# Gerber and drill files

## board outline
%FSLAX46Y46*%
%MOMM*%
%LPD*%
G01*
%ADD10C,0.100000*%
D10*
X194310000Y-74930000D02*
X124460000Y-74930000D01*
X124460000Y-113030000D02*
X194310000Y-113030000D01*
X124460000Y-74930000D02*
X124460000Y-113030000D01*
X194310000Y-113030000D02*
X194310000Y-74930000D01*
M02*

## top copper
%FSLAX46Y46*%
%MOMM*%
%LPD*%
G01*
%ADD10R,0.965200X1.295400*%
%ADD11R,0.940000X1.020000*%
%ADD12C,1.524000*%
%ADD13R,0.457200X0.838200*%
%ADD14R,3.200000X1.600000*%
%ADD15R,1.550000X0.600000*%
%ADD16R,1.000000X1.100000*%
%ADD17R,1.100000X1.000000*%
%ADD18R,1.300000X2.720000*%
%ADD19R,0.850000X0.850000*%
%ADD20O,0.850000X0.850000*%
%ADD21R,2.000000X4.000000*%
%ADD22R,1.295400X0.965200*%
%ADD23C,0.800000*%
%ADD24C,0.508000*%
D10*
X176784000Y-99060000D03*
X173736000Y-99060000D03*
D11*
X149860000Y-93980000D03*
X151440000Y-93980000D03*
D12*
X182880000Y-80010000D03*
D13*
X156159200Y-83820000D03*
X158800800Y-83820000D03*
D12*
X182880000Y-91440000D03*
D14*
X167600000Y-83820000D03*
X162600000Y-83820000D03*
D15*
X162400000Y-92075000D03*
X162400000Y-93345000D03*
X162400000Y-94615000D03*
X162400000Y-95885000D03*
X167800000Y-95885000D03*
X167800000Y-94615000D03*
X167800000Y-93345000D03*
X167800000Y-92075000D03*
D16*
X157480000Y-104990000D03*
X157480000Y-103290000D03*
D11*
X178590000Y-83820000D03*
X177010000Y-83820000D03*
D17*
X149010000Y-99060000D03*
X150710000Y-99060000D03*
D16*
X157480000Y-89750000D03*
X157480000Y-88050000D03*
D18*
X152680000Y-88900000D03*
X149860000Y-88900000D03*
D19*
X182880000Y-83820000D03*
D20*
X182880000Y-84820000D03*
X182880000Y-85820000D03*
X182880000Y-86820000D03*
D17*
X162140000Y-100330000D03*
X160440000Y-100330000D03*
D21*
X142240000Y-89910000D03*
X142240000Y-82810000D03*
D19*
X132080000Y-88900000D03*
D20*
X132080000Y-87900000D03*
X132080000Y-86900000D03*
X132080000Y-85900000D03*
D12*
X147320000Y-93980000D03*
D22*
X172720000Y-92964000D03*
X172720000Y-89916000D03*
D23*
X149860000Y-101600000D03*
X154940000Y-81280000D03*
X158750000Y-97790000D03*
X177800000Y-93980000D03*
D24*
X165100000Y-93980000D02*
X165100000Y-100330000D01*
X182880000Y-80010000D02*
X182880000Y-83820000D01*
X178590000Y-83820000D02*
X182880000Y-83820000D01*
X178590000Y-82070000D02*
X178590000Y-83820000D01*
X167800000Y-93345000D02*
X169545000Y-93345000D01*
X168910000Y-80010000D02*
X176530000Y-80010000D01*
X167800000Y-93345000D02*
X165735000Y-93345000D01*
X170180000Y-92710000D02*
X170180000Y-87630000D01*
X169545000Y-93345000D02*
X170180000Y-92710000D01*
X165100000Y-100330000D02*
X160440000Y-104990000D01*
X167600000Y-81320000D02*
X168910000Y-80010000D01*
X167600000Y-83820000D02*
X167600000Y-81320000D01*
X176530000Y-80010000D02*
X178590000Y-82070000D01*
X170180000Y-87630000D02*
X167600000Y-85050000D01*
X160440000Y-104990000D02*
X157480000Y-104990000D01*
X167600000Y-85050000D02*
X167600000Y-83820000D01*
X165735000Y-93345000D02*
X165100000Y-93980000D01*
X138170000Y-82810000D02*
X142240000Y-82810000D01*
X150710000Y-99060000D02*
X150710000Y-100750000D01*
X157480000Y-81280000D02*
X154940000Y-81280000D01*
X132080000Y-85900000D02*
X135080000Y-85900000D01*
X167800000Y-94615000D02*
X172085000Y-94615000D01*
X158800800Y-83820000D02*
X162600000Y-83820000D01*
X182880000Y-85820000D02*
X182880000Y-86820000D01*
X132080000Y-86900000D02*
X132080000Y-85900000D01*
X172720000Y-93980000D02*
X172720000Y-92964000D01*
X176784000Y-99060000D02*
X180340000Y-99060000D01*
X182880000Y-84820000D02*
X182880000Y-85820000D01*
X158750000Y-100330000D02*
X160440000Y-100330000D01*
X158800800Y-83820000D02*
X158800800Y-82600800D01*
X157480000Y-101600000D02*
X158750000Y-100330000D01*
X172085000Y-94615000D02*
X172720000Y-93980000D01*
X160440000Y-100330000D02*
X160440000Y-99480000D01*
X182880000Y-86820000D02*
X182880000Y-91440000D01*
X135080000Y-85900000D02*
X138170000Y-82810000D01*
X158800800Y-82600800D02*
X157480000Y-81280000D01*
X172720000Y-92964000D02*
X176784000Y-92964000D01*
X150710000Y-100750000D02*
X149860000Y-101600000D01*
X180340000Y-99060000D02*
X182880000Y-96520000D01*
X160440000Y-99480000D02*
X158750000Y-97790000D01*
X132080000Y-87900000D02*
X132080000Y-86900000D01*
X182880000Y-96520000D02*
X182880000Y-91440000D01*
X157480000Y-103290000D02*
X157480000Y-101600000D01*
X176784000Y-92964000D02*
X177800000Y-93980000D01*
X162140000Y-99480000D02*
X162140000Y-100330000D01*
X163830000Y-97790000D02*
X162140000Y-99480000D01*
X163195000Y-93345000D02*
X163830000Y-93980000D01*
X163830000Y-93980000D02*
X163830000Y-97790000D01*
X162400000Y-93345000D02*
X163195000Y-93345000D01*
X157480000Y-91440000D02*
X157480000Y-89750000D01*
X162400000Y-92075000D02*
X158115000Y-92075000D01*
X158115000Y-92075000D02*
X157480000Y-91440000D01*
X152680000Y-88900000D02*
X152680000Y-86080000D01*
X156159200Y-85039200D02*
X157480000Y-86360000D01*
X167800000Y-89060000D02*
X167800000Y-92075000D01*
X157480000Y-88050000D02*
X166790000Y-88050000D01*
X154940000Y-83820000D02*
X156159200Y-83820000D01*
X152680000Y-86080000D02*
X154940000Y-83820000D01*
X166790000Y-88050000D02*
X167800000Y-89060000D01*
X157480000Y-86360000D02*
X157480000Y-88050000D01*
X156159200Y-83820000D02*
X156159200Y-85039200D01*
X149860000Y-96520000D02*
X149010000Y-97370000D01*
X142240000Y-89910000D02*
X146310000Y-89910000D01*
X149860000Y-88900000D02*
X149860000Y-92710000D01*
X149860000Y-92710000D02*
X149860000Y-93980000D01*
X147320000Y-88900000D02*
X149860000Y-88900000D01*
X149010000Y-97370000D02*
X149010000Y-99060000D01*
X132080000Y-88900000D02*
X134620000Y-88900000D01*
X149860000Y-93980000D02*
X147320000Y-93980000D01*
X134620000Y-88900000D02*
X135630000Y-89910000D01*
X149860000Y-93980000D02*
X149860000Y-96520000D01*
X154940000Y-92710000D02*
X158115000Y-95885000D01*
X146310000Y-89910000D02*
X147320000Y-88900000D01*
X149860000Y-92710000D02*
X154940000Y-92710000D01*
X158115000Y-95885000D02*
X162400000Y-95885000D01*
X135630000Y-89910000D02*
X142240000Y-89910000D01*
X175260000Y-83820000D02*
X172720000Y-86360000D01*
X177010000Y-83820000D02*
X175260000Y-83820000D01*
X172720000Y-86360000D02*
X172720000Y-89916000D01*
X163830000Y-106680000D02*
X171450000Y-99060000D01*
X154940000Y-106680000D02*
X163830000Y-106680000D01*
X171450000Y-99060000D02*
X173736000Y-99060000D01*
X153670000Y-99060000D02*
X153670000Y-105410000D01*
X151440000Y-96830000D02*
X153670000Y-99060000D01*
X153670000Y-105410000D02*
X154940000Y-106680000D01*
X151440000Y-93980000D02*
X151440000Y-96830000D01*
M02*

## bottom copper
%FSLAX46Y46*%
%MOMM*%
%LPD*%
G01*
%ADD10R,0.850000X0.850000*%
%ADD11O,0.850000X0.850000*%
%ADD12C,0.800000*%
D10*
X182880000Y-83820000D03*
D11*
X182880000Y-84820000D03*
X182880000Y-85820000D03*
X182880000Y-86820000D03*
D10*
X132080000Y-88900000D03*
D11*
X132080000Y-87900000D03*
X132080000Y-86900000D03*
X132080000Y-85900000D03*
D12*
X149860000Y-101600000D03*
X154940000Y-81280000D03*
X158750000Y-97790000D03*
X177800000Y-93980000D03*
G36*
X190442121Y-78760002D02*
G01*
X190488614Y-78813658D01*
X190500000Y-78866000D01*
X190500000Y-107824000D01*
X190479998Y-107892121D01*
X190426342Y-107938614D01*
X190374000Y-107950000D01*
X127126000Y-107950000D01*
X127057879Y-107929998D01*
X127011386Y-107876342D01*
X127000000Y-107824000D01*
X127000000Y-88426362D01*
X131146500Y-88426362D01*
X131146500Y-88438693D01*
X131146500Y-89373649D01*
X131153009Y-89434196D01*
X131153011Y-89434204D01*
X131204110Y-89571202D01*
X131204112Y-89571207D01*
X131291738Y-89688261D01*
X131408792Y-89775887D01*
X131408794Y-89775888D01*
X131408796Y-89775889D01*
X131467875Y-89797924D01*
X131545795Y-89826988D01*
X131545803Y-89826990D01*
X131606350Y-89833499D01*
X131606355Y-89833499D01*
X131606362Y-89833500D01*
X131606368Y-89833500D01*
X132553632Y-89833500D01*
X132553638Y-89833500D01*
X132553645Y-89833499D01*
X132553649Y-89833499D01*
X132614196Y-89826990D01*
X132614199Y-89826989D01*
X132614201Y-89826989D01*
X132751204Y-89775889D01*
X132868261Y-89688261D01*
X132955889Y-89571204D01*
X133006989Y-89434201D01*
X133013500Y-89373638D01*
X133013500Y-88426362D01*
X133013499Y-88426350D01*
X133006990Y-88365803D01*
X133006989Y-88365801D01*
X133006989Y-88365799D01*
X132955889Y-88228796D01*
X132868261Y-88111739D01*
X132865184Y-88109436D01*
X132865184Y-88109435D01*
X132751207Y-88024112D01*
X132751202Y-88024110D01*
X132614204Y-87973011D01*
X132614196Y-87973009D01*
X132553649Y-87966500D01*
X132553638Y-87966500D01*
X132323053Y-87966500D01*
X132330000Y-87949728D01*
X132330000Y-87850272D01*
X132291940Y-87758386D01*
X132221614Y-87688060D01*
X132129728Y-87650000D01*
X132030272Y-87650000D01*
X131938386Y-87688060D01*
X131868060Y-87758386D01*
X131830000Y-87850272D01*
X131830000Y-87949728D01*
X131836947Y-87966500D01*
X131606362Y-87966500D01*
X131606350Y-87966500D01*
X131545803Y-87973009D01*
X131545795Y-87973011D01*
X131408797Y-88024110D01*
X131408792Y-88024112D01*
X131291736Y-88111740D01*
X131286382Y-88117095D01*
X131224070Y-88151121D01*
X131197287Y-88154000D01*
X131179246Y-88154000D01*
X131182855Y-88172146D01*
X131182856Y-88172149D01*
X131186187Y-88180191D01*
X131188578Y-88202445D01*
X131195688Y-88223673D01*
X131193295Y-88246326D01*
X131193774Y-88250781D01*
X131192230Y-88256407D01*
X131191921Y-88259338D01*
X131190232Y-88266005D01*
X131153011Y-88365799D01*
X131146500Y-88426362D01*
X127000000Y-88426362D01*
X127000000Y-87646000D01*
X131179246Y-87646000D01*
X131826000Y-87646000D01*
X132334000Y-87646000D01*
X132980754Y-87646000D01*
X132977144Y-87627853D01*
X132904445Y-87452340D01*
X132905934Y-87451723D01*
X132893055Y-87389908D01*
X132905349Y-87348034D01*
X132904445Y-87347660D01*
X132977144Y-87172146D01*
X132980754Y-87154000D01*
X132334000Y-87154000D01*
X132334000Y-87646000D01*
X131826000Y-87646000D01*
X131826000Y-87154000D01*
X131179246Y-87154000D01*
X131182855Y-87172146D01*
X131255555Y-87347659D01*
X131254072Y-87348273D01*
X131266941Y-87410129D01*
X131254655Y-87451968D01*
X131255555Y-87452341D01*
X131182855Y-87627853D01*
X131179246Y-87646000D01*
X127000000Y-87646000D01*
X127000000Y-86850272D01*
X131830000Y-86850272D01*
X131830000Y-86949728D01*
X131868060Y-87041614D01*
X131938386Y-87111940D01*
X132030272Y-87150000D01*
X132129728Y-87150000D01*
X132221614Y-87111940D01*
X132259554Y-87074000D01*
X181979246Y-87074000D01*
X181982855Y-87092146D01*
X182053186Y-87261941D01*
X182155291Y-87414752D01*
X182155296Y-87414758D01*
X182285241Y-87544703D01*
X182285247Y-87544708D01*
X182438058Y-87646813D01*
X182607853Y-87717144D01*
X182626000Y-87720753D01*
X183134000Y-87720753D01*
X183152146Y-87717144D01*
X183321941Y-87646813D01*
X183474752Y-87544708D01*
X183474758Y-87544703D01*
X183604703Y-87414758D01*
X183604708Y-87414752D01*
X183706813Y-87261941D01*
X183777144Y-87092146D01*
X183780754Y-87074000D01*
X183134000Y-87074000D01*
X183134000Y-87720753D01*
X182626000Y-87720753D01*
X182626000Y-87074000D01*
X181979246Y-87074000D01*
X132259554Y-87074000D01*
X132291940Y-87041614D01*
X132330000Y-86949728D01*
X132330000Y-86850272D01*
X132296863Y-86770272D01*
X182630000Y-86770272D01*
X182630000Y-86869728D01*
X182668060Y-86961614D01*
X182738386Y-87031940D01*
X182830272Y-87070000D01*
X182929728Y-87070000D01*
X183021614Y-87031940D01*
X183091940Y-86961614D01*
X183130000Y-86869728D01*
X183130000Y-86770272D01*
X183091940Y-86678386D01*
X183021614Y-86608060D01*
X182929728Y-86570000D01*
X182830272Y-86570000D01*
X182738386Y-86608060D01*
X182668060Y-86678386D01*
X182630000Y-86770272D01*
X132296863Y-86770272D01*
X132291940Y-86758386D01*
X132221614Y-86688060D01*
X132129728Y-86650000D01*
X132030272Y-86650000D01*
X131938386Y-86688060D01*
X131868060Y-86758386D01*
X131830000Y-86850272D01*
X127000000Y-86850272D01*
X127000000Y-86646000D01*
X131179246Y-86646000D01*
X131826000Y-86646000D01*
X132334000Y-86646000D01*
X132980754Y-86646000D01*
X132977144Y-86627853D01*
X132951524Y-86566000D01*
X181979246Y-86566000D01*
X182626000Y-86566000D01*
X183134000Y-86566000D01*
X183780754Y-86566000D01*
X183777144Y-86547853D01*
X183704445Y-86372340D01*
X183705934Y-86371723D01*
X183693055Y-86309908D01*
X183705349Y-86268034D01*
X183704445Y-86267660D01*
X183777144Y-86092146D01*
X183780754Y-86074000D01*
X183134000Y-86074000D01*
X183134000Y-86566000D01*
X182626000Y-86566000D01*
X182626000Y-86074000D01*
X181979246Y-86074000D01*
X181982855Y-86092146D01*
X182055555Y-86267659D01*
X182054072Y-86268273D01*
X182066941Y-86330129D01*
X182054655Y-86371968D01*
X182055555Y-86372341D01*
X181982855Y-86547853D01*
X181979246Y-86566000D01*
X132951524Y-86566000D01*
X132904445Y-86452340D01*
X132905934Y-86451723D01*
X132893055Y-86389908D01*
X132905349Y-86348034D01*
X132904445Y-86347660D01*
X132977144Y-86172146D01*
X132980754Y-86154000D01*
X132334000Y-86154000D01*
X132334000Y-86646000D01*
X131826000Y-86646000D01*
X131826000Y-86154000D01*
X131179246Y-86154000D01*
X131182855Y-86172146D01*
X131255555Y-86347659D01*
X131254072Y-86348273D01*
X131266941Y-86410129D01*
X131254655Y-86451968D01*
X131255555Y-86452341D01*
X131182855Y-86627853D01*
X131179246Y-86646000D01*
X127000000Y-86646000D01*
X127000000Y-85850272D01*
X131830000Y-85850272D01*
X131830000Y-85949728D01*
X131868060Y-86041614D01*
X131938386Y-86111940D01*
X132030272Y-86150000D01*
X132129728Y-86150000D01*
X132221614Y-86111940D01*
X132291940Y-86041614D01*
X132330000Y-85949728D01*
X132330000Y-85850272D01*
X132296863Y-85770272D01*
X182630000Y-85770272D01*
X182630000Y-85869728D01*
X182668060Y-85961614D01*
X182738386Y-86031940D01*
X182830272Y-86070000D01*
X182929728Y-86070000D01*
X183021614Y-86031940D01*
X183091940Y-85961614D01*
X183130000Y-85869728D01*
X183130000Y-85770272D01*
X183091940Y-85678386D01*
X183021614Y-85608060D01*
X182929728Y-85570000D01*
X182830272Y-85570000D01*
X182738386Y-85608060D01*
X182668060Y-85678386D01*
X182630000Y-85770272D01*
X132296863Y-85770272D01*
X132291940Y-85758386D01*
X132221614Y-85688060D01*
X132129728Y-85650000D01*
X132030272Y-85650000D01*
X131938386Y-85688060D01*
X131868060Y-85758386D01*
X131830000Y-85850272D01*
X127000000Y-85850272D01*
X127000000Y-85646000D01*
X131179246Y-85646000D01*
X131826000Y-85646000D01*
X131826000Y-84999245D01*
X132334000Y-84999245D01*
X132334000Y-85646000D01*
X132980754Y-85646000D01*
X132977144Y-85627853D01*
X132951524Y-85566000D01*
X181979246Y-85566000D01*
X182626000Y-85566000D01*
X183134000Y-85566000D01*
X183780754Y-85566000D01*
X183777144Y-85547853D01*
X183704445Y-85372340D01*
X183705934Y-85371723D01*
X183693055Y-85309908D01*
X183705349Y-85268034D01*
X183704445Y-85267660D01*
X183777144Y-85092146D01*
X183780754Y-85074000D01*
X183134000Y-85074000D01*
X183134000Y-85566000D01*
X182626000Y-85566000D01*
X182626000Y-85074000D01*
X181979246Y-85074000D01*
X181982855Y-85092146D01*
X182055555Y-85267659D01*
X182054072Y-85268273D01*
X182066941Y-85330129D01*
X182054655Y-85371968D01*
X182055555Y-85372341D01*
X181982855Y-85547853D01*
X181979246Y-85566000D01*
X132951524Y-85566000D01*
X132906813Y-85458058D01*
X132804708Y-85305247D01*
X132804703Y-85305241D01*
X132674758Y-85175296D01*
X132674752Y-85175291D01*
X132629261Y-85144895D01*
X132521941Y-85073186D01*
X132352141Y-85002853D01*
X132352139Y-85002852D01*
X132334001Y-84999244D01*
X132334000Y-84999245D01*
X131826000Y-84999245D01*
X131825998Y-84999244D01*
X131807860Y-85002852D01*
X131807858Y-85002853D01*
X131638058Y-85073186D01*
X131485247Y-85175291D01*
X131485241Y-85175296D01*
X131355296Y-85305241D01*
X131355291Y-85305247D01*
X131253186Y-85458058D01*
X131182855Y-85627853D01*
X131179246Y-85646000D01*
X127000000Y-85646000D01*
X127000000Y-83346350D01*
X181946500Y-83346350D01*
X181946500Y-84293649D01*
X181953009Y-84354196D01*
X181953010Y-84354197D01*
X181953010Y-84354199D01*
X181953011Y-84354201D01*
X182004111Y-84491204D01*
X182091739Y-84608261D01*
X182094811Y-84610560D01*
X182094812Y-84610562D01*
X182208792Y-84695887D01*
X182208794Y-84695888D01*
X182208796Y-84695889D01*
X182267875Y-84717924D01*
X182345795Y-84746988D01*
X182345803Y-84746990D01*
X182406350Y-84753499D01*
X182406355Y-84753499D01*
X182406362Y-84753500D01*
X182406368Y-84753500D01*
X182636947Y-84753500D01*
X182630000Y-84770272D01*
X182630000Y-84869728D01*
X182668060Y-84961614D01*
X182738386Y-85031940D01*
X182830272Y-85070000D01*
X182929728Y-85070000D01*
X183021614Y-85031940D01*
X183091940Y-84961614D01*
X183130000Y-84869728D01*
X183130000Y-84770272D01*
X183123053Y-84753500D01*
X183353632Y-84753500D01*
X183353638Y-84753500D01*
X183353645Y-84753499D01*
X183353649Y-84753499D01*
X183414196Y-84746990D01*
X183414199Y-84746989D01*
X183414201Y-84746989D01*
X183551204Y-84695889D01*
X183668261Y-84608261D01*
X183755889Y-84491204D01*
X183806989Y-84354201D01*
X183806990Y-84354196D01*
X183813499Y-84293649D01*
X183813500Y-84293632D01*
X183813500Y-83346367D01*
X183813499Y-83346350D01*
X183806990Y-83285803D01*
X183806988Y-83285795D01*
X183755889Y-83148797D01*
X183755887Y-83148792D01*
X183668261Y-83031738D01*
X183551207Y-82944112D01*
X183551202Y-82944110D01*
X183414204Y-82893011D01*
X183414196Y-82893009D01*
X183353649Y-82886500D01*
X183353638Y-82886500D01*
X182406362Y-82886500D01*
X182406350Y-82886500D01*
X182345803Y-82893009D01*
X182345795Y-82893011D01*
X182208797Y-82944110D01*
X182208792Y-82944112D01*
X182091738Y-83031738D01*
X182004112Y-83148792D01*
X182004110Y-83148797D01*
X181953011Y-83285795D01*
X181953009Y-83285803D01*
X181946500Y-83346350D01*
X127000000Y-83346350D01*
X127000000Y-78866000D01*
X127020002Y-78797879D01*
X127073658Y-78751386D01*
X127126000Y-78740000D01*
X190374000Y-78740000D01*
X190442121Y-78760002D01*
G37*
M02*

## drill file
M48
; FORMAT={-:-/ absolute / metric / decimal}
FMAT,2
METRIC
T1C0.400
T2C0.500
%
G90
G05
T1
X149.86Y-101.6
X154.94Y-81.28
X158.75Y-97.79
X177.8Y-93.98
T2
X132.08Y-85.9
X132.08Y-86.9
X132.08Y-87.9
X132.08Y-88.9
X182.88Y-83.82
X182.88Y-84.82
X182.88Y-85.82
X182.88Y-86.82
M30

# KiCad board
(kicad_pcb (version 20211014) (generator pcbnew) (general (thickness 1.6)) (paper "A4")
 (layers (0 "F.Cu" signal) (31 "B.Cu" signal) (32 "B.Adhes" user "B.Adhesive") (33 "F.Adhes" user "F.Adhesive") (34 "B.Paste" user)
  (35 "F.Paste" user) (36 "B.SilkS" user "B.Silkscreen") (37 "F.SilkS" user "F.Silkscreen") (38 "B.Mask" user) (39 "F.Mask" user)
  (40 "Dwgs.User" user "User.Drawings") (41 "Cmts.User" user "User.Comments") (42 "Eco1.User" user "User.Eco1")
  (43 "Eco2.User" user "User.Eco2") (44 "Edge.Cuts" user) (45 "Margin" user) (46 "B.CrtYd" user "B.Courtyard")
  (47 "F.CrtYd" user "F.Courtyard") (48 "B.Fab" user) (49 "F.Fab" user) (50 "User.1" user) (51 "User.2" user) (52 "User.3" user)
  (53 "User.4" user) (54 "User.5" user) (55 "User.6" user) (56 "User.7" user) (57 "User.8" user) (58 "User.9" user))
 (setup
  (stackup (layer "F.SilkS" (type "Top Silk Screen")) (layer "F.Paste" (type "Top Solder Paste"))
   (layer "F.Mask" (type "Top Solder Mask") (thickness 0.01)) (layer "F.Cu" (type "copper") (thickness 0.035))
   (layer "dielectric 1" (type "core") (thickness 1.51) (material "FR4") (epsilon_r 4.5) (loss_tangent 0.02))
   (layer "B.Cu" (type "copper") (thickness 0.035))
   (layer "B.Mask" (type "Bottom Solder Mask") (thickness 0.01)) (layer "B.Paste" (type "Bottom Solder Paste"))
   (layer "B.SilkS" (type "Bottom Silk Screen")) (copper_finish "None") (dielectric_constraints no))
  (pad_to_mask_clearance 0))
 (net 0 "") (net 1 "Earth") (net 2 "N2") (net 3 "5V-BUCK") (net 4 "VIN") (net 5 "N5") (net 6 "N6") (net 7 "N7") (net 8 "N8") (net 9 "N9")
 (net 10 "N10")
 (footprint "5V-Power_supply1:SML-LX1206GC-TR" (layer "F.Cu") (at 175.26 99.06 180)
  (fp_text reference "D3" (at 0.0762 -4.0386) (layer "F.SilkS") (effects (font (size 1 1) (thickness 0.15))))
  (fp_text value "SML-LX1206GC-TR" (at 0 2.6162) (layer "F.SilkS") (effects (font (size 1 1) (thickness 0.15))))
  (pad "1" smd rect (at -1.524 0 180) (size 0.9652 1.2954) (layers "F.Cu" "F.Paste" "F.Mask") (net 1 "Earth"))
  (pad "2" smd rect (at 1.524 0 180) (size 0.9652 1.2954) (layers "F.Cu" "F.Paste" "F.Mask") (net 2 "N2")))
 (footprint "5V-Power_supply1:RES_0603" (layer "F.Cu") (at 150.65 93.98)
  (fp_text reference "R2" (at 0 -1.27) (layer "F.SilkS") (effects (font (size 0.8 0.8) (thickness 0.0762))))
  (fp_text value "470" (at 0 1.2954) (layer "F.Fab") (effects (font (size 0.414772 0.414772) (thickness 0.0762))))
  (pad "1" smd rect (at -0.79 0) (size 0.94 1.02) (layers "F.Cu" "F.Paste" "F.Mask") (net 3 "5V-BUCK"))
  (pad "2" smd rect (at 0.79 0) (size 0.94 1.02) (layers "F.Cu" "F.Paste" "F.Mask") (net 2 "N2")))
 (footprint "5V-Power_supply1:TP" (layer "F.Cu") (at 182.88 80.01 90)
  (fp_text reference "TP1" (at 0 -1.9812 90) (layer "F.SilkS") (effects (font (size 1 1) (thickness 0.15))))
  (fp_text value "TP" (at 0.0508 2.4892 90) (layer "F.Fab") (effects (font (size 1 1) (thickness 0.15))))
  (pad "1" smd circle (at 0 0 90) (size 1.524 1.524) (layers "F.Cu" "F.Paste" "F.Mask") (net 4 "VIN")))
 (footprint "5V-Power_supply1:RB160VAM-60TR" (layer "F.Cu") (at 157.48 83.82)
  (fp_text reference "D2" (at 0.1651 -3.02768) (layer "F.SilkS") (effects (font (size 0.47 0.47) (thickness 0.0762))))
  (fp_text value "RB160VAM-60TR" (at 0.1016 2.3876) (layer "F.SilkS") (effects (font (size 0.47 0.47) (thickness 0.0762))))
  (pad "1" smd rect (at -1.3208 0) (size 0.4572 0.8382) (layers "F.Cu" "F.Paste" "F.Mask") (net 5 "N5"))
  (pad "2" smd rect (at 1.3208 0) (size 0.4572 0.8382) (layers "F.Cu" "F.Paste" "F.Mask") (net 1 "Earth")))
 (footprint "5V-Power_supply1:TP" (layer "F.Cu") (at 182.88 91.44)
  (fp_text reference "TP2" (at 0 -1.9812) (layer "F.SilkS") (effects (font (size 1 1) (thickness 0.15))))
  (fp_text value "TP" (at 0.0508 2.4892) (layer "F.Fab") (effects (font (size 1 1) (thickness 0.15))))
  (pad "1" smd circle (at 0 0) (size 1.524 1.524) (layers "F.Cu" "F.Paste" "F.Mask") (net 1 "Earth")))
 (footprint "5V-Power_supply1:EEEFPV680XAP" (layer "F.Cu") (at 165.1 83.82 180)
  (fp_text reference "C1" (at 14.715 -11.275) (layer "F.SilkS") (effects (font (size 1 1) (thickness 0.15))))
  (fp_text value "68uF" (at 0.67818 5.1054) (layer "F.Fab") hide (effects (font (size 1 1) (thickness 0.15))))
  (pad "1" smd rect (at -2.5 0 180) (size 3.2 1.6) (layers "F.Cu" "F.Paste" "F.Mask") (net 4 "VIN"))
  (pad "2" smd rect (at 2.5 0 180) (size 3.2 1.6) (layers "F.Cu" "F.Paste" "F.Mask") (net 1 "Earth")))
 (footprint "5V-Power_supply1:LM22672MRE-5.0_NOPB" (layer "F.Cu") (at 165.1 93.98)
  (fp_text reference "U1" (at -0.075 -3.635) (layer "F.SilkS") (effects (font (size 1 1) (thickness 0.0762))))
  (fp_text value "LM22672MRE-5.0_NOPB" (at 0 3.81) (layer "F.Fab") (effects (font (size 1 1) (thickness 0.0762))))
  (pad "1" smd rect (at -2.7 -1.905) (size 1.55 0.6) (layers "F.Cu" "F.Paste") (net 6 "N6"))
  (pad "2" smd rect (at -2.7 -0.635) (size 1.55 0.6) (layers "F.Cu" "F.Paste") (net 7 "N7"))
  (pad "3" smd rect (at -2.7 0.635) (size 1.55 0.6) (layers "F.Cu" "F.Paste") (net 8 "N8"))
  (pad "4" smd rect (at -2.7 1.905) (size 1.55 0.6) (layers "F.Cu" "F.Paste") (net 3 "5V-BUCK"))
  (pad "5" smd rect (at 2.7 1.905) (size 1.55 0.6) (layers "F.Cu" "F.Paste") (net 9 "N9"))
  (pad "6" smd rect (at 2.7 0.635) (size 1.55 0.6) (layers "F.Cu" "F.Paste") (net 1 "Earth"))
  (pad "7" smd rect (at 2.7 -0.635) (size 1.55 0.6) (layers "F.Cu" "F.Paste") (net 4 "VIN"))
  (pad "8" smd rect (at 2.7 -1.905) (size 1.55 0.6) (layers "F.Cu" "F.Paste") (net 5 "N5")))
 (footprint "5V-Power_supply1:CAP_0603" (layer "F.Cu") (at 157.48 104.14 90)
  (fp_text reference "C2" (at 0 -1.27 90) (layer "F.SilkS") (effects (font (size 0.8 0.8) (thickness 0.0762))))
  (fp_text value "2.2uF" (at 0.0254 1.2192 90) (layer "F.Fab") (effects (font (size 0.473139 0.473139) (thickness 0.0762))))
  (pad "1" smd rect (at -0.85 0 90) (size 1.1 1) (layers "F.Cu" "F.Paste" "F.Mask") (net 4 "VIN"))
  (pad "2" smd rect (at 0.85 0 90) (size 1.1 1) (layers "F.Cu" "F.Paste" "F.Mask") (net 1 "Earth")))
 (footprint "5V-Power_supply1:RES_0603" (layer "F.Cu") (at 177.8 83.82 180)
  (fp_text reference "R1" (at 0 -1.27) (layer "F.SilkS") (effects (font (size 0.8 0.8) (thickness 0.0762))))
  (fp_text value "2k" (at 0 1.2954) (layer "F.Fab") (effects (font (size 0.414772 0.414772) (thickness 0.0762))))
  (pad "1" smd rect (at -0.79 0 180) (size 0.94 1.02) (layers "F.Cu" "F.Paste" "F.Mask") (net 4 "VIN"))
  (pad "2" smd rect (at 0.79 0 180) (size 0.94 1.02) (layers "F.Cu" "F.Paste" "F.Mask") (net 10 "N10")))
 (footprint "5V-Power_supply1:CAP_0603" (layer "F.Cu") (at 149.86 99.06)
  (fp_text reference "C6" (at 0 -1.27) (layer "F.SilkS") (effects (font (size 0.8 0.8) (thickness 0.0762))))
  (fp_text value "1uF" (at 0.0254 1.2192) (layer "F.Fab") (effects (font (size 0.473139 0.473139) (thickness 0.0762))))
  (pad "1" smd rect (at -0.85 0) (size 1.1 1) (layers "F.Cu" "F.Paste" "F.Mask") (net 3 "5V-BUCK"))
  (pad "2" smd rect (at 0.85 0) (size 1.1 1) (layers "F.Cu" "F.Paste" "F.Mask") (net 1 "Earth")))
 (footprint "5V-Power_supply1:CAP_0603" (layer "F.Cu") (at 157.48 88.9 90)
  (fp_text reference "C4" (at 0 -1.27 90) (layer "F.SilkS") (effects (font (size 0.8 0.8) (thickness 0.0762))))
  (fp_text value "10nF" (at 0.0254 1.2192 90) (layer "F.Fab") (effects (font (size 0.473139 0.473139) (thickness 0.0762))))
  (pad "1" smd rect (at -0.85 0 90) (size 1.1 1) (layers "F.Cu" "F.Paste" "F.Mask") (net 6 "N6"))
  (pad "2" smd rect (at 0.85 0 90) (size 1.1 1) (layers "F.Cu" "F.Paste" "F.Mask") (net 5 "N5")))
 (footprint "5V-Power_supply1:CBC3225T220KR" (layer "F.Cu") (at 151.27 88.9 180)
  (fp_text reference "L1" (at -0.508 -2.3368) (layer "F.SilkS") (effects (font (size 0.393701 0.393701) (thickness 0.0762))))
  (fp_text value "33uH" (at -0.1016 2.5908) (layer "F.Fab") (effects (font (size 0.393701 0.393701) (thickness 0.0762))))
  (pad "1" smd rect (at -1.41 0 180) (size 1.3 2.72) (layers "F.Cu" "F.Paste" "F.Mask") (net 5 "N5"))
  (pad "2" smd rect (at 1.41 0 180) (size 1.3 2.72) (layers "F.Cu" "F.Paste" "F.Mask") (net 3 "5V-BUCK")))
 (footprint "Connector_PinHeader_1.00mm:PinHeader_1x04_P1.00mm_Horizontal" (layer "F.Cu") (at 182.88 83.82)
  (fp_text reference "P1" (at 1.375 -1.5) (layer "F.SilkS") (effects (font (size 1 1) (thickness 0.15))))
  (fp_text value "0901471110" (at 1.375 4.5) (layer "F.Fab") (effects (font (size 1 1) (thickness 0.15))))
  (pad "1" thru_hole rect (at 0 0) (size 0.85 0.85) (drill 0.5) (layers *.Cu *.Mask) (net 4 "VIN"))
  (pad "2" thru_hole oval (at 0 1) (size 0.85 0.85) (drill 0.5) (layers *.Cu *.Mask) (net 1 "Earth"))
  (pad "3" thru_hole oval (at 0 2) (size 0.85 0.85) (drill 0.5) (layers *.Cu *.Mask) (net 1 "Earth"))
  (pad "4" thru_hole oval (at 0 3) (size 0.85 0.85) (drill 0.5) (layers *.Cu *.Mask) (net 1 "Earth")))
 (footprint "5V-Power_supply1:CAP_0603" (layer "F.Cu") (at 161.29 100.33 180)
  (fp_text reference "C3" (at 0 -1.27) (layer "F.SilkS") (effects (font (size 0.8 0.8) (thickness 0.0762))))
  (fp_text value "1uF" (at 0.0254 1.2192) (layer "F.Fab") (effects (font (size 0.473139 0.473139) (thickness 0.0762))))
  (pad "1" smd rect (at -0.85 0 180) (size 1.1 1) (layers "F.Cu" "F.Paste" "F.Mask") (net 7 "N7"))
  (pad "2" smd rect (at 0.85 0 180) (size 1.1 1) (layers "F.Cu" "F.Paste" "F.Mask") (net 1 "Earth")))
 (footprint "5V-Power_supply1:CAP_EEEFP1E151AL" (layer "F.Cu") (at 142.24 86.36 90)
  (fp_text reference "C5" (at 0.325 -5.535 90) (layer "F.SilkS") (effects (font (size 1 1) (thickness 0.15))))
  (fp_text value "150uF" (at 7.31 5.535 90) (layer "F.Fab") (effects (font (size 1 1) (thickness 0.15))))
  (pad "1" smd rect (at -3.55 0 90) (size 4 2) (layers "F.Cu" "F.Paste" "F.Mask") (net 3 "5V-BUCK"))
  (pad "2" smd rect (at 3.55 0 90) (size 4 2) (layers "F.Cu" "F.Paste" "F.Mask") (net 1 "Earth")))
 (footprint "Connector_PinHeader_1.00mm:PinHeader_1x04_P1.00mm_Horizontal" (layer "F.Cu") (at 132.08 88.9 180)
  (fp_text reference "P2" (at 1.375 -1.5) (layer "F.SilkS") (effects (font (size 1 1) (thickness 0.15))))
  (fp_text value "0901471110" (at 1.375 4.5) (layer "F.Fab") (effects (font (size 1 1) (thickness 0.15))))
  (pad "1" thru_hole rect (at 0 0 180) (size 0.85 0.85) (drill 0.5) (layers *.Cu *.Mask) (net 3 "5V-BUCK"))
  (pad "2" thru_hole oval (at 0 1 180) (size 0.85 0.85) (drill 0.5) (layers *.Cu *.Mask) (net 1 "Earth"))
  (pad "3" thru_hole oval (at 0 2 180) (size 0.85 0.85) (drill 0.5) (layers *.Cu *.Mask) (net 1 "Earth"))
  (pad "4" thru_hole oval (at 0 3 180) (size 0.85 0.85) (drill 0.5) (layers *.Cu *.Mask) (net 1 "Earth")))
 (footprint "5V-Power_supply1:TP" (layer "F.Cu") (at 147.32 93.98)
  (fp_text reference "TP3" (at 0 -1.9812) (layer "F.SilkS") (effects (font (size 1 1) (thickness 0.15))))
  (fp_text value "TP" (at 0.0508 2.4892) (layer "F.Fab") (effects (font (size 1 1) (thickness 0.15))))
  (pad "1" smd circle (at 0 0) (size 1.524 1.524) (layers "F.Cu" "F.Paste" "F.Mask") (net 3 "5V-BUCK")))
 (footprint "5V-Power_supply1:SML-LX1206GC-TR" (layer "F.Cu") (at 172.72 91.44 90)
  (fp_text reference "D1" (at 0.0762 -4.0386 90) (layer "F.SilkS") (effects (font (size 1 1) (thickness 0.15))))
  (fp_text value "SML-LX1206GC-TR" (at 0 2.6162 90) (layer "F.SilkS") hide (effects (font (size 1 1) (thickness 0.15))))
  (pad "1" smd rect (at -1.524 0 90) (size 0.9652 1.2954) (layers "F.Cu" "F.Paste" "F.Mask") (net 1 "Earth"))
  (pad "2" smd rect (at 1.524 0 90) (size 0.9652 1.2954) (layers "F.Cu" "F.Paste" "F.Mask") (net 10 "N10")))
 (gr_line (start 194.31 74.93) (end 124.46 74.93) (layer "Edge.Cuts") (width 0.1))
 (gr_line (start 124.46 113.03) (end 194.31 113.03) (layer "Edge.Cuts") (width 0.1))
 (gr_line (start 124.46 74.93) (end 124.46 113.03) (layer "Edge.Cuts") (width 0.1))
 (gr_line (start 194.31 113.03) (end 194.31 74.93) (layer "Edge.Cuts") (width 0.1))
 (segment (start 165.1 93.98) (end 165.1 100.33) (width 0.508) (layer "F.Cu") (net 4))
 (segment (start 182.88 80.01) (end 182.88 83.82) (width 0.508) (layer "F.Cu") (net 4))
 (segment (start 178.59 83.82) (end 182.88 83.82) (width 0.508) (layer "F.Cu") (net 4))
 (segment (start 178.59 82.07) (end 178.59 83.82) (width 0.508) (layer "F.Cu") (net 4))
 (segment (start 167.8 93.345) (end 169.545 93.345) (width 0.508) (layer "F.Cu") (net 4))
 (segment (start 168.91 80.01) (end 176.53 80.01) (width 0.508) (layer "F.Cu") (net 4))
 (segment (start 167.8 93.345) (end 165.735 93.345) (width 0.508) (layer "F.Cu") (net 4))
 (segment (start 170.18 92.71) (end 170.18 87.63) (width 0.508) (layer "F.Cu") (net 4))
 (segment (start 169.545 93.345) (end 170.18 92.71) (width 0.508) (layer "F.Cu") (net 4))
 (segment (start 165.1 100.33) (end 160.44 104.99) (width 0.508) (layer "F.Cu") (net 4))
 (segment (start 167.6 81.32) (end 168.91 80.01) (width 0.508) (layer "F.Cu") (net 4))
 (segment (start 167.6 83.82) (end 167.6 81.32) (width 0.508) (layer "F.Cu") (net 4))
 (segment (start 176.53 80.01) (end 178.59 82.07) (width 0.508) (layer "F.Cu") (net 4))
 (segment (start 170.18 87.63) (end 167.6 85.05) (width 0.508) (layer "F.Cu") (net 4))
 (segment (start 160.44 104.99) (end 157.48 104.99) (width 0.508) (layer "F.Cu") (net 4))
 (segment (start 167.6 85.05) (end 167.6 83.82) (width 0.508) (layer "F.Cu") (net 4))
 (segment (start 165.735 93.345) (end 165.1 93.98) (width 0.508) (layer "F.Cu") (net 4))
 (segment (start 138.17 82.81) (end 142.24 82.81) (width 0.508) (layer "F.Cu") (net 1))
 (segment (start 150.71 99.06) (end 150.71 100.75) (width 0.508) (layer "F.Cu") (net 1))
 (segment (start 157.48 81.28) (end 154.94 81.28) (width 0.508) (layer "F.Cu") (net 1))
 (segment (start 132.08 85.9) (end 135.08 85.9) (width 0.508) (layer "F.Cu") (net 1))
 (segment (start 167.8 94.615) (end 172.085 94.615) (width 0.508) (layer "F.Cu") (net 1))
 (segment (start 158.8008 83.82) (end 162.6 83.82) (width 0.508) (layer "F.Cu") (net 1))
 (segment (start 182.88 85.82) (end 182.88 86.82) (width 0.508) (layer "F.Cu") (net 1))
 (segment (start 132.08 86.9) (end 132.08 85.9) (width 0.508) (layer "F.Cu") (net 1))
 (segment (start 172.72 93.98) (end 172.72 92.964) (width 0.508) (layer "F.Cu") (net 1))
 (segment (start 176.784 99.06) (end 180.34 99.06) (width 0.508) (layer "F.Cu") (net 1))
 (segment (start 182.88 84.82) (end 182.88 85.82) (width 0.508) (layer "F.Cu") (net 1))
 (segment (start 158.75 100.33) (end 160.44 100.33) (width 0.508) (layer "F.Cu") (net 1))
 (segment (start 158.8008 83.82) (end 158.8008 82.6008) (width 0.508) (layer "F.Cu") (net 1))
 (segment (start 157.48 101.6) (end 158.75 100.33) (width 0.508) (layer "F.Cu") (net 1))
 (segment (start 172.085 94.615) (end 172.72 93.98) (width 0.508) (layer "F.Cu") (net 1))
 (segment (start 160.44 100.33) (end 160.44 99.48) (width 0.508) (layer "F.Cu") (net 1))
 (segment (start 182.88 86.82) (end 182.88 91.44) (width 0.508) (layer "F.Cu") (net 1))
 (segment (start 135.08 85.9) (end 138.17 82.81) (width 0.508) (layer "F.Cu") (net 1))
 (segment (start 158.8008 82.6008) (end 157.48 81.28) (width 0.508) (layer "F.Cu") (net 1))
 (segment (start 172.72 92.964) (end 176.784 92.964) (width 0.508) (layer "F.Cu") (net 1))
 (segment (start 150.71 100.75) (end 149.86 101.6) (width 0.508) (layer "F.Cu") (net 1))
 (segment (start 180.34 99.06) (end 182.88 96.52) (width 0.508) (layer "F.Cu") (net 1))
 (segment (start 160.44 99.48) (end 158.75 97.79) (width 0.508) (layer "F.Cu") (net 1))
 (segment (start 132.08 87.9) (end 132.08 86.9) (width 0.508) (layer "F.Cu") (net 1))
 (segment (start 182.88 96.52) (end 182.88 91.44) (width 0.508) (layer "F.Cu") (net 1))
 (segment (start 157.48 103.29) (end 157.48 101.6) (width 0.508) (layer "F.Cu") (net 1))
 (segment (start 176.784 92.964) (end 177.8 93.98) (width 0.508) (layer "F.Cu") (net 1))
 (via (at 149.86 101.6) (size 0.8) (drill 0.4) (layers "F.Cu" "B.Cu") (free) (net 1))
 (via (at 154.94 81.28) (size 0.8) (drill 0.4) (layers "F.Cu" "B.Cu") (free) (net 1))
 (via (at 158.75 97.79) (size 0.8) (drill 0.4) (layers "F.Cu" "B.Cu") (free) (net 1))
 (via (at 177.8 93.98) (size 0.8) (drill 0.4) (layers "F.Cu" "B.Cu") (free) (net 1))
 (segment (start 162.14 99.48) (end 162.14 100.33) (width 0.508) (layer "F.Cu") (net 7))
 (segment (start 163.83 97.79) (end 162.14 99.48) (width 0.508) (layer "F.Cu") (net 7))
 (segment (start 163.195 93.345) (end 163.83 93.98) (width 0.508) (layer "F.Cu") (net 7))
 (segment (start 163.83 93.98) (end 163.83 97.79) (width 0.508) (layer "F.Cu") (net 7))
 (segment (start 162.4 93.345) (end 163.195 93.345) (width 0.508) (layer "F.Cu") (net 7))
 (segment (start 157.48 91.44) (end 157.48 89.75) (width 0.508) (layer "F.Cu") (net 6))
 (segment (start 162.4 92.075) (end 158.115 92.075) (width 0.508) (layer "F.Cu") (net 6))
 (segment (start 158.115 92.075) (end 157.48 91.44) (width 0.508) (layer "F.Cu") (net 6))
 (segment (start 152.68 88.9) (end 152.68 86.08) (width 0.508) (layer "F.Cu") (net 5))
 (segment (start 156.1592 85.0392) (end 157.48 86.36) (width 0.508) (layer "F.Cu") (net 5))
 (segment (start 167.8 89.06) (end 167.8 92.075) (width 0.508) (layer "F.Cu") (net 5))
 (segment (start 157.48 88.05) (end 166.79 88.05) (width 0.508) (layer "F.Cu") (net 5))
 (segment (start 154.94 83.82) (end 156.1592 83.82) (width 0.508) (layer "F.Cu") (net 5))
 (segment (start 152.68 86.08) (end 154.94 83.82) (width 0.508) (layer "F.Cu") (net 5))
 (segment (start 166.79 88.05) (end 167.8 89.06) (width 0.508) (layer "F.Cu") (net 5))
 (segment (start 157.48 86.36) (end 157.48 88.05) (width 0.508) (layer "F.Cu") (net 5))
 (segment (start 156.1592 83.82) (end 156.1592 85.0392) (width 0.508) (layer "F.Cu") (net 5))
 (segment (start 149.86 96.52) (end 149.01 97.37) (width 0.508) (layer "F.Cu") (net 3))
 (segment (start 142.24 89.91) (end 146.31 89.91) (width 0.508) (layer "F.Cu") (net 3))
 (segment (start 149.86 88.9) (end 149.86 92.71) (width 0.508) (layer "F.Cu") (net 3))
 (segment (start 149.86 92.71) (end 149.86 93.98) (width 0.508) (layer "F.Cu") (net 3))
 (segment (start 147.32 88.9) (end 149.86 88.9) (width 0.508) (layer "F.Cu") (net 3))
 (segment (start 149.01 97.37) (end 149.01 99.06) (width 0.508) (layer "F.Cu") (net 3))
 (segment (start 132.08 88.9) (end 134.62 88.9) (width 0.508) (layer "F.Cu") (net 3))
 (segment (start 149.86 93.98) (end 147.32 93.98) (width 0.508) (layer "F.Cu") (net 3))
 (segment (start 134.62 88.9) (end 135.63 89.91) (width 0.508) (layer "F.Cu") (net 3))
 (segment (start 149.86 93.98) (end 149.86 96.52) (width 0.508) (layer "F.Cu") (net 3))
 (segment (start 154.94 92.71) (end 158.115 95.885) (width 0.508) (layer "F.Cu") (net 3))
 (segment (start 146.31 89.91) (end 147.32 88.9) (width 0.508) (layer "F.Cu") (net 3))
 (segment (start 149.86 92.71) (end 154.94 92.71) (width 0.508) (layer "F.Cu") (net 3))
 (segment (start 158.115 95.885) (end 162.4 95.885) (width 0.508) (layer "F.Cu") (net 3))
 (segment (start 135.63 89.91) (end 142.24 89.91) (width 0.508) (layer "F.Cu") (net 3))
 (segment (start 175.26 83.82) (end 172.72 86.36) (width 0.508) (layer "F.Cu") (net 10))
 (segment (start 177.01 83.82) (end 175.26 83.82) (width 0.508) (layer "F.Cu") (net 10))
 (segment (start 172.72 86.36) (end 172.72 89.916) (width 0.508) (layer "F.Cu") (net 10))
 (segment (start 163.83 106.68) (end 171.45 99.06) (width 0.508) (layer "F.Cu") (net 2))
 (segment (start 154.94 106.68) (end 163.83 106.68) (width 0.508) (layer "F.Cu") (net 2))
 (segment (start 171.45 99.06) (end 173.736 99.06) (width 0.508) (layer "F.Cu") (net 2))
 (segment (start 153.67 99.06) (end 153.67 105.41) (width 0.508) (layer "F.Cu") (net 2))
 (segment (start 151.44 96.83) (end 153.67 99.06) (width 0.508) (layer "F.Cu") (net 2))
 (segment (start 153.67 105.41) (end 154.94 106.68) (width 0.508) (layer "F.Cu") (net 2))
 (segment (start 151.44 93.98) (end 151.44 96.83) (width 0.508) (layer "F.Cu") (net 2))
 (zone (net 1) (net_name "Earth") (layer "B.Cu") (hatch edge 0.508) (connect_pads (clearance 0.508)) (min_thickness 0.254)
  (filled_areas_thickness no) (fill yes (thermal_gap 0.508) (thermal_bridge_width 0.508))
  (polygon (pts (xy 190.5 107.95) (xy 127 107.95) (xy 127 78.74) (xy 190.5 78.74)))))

